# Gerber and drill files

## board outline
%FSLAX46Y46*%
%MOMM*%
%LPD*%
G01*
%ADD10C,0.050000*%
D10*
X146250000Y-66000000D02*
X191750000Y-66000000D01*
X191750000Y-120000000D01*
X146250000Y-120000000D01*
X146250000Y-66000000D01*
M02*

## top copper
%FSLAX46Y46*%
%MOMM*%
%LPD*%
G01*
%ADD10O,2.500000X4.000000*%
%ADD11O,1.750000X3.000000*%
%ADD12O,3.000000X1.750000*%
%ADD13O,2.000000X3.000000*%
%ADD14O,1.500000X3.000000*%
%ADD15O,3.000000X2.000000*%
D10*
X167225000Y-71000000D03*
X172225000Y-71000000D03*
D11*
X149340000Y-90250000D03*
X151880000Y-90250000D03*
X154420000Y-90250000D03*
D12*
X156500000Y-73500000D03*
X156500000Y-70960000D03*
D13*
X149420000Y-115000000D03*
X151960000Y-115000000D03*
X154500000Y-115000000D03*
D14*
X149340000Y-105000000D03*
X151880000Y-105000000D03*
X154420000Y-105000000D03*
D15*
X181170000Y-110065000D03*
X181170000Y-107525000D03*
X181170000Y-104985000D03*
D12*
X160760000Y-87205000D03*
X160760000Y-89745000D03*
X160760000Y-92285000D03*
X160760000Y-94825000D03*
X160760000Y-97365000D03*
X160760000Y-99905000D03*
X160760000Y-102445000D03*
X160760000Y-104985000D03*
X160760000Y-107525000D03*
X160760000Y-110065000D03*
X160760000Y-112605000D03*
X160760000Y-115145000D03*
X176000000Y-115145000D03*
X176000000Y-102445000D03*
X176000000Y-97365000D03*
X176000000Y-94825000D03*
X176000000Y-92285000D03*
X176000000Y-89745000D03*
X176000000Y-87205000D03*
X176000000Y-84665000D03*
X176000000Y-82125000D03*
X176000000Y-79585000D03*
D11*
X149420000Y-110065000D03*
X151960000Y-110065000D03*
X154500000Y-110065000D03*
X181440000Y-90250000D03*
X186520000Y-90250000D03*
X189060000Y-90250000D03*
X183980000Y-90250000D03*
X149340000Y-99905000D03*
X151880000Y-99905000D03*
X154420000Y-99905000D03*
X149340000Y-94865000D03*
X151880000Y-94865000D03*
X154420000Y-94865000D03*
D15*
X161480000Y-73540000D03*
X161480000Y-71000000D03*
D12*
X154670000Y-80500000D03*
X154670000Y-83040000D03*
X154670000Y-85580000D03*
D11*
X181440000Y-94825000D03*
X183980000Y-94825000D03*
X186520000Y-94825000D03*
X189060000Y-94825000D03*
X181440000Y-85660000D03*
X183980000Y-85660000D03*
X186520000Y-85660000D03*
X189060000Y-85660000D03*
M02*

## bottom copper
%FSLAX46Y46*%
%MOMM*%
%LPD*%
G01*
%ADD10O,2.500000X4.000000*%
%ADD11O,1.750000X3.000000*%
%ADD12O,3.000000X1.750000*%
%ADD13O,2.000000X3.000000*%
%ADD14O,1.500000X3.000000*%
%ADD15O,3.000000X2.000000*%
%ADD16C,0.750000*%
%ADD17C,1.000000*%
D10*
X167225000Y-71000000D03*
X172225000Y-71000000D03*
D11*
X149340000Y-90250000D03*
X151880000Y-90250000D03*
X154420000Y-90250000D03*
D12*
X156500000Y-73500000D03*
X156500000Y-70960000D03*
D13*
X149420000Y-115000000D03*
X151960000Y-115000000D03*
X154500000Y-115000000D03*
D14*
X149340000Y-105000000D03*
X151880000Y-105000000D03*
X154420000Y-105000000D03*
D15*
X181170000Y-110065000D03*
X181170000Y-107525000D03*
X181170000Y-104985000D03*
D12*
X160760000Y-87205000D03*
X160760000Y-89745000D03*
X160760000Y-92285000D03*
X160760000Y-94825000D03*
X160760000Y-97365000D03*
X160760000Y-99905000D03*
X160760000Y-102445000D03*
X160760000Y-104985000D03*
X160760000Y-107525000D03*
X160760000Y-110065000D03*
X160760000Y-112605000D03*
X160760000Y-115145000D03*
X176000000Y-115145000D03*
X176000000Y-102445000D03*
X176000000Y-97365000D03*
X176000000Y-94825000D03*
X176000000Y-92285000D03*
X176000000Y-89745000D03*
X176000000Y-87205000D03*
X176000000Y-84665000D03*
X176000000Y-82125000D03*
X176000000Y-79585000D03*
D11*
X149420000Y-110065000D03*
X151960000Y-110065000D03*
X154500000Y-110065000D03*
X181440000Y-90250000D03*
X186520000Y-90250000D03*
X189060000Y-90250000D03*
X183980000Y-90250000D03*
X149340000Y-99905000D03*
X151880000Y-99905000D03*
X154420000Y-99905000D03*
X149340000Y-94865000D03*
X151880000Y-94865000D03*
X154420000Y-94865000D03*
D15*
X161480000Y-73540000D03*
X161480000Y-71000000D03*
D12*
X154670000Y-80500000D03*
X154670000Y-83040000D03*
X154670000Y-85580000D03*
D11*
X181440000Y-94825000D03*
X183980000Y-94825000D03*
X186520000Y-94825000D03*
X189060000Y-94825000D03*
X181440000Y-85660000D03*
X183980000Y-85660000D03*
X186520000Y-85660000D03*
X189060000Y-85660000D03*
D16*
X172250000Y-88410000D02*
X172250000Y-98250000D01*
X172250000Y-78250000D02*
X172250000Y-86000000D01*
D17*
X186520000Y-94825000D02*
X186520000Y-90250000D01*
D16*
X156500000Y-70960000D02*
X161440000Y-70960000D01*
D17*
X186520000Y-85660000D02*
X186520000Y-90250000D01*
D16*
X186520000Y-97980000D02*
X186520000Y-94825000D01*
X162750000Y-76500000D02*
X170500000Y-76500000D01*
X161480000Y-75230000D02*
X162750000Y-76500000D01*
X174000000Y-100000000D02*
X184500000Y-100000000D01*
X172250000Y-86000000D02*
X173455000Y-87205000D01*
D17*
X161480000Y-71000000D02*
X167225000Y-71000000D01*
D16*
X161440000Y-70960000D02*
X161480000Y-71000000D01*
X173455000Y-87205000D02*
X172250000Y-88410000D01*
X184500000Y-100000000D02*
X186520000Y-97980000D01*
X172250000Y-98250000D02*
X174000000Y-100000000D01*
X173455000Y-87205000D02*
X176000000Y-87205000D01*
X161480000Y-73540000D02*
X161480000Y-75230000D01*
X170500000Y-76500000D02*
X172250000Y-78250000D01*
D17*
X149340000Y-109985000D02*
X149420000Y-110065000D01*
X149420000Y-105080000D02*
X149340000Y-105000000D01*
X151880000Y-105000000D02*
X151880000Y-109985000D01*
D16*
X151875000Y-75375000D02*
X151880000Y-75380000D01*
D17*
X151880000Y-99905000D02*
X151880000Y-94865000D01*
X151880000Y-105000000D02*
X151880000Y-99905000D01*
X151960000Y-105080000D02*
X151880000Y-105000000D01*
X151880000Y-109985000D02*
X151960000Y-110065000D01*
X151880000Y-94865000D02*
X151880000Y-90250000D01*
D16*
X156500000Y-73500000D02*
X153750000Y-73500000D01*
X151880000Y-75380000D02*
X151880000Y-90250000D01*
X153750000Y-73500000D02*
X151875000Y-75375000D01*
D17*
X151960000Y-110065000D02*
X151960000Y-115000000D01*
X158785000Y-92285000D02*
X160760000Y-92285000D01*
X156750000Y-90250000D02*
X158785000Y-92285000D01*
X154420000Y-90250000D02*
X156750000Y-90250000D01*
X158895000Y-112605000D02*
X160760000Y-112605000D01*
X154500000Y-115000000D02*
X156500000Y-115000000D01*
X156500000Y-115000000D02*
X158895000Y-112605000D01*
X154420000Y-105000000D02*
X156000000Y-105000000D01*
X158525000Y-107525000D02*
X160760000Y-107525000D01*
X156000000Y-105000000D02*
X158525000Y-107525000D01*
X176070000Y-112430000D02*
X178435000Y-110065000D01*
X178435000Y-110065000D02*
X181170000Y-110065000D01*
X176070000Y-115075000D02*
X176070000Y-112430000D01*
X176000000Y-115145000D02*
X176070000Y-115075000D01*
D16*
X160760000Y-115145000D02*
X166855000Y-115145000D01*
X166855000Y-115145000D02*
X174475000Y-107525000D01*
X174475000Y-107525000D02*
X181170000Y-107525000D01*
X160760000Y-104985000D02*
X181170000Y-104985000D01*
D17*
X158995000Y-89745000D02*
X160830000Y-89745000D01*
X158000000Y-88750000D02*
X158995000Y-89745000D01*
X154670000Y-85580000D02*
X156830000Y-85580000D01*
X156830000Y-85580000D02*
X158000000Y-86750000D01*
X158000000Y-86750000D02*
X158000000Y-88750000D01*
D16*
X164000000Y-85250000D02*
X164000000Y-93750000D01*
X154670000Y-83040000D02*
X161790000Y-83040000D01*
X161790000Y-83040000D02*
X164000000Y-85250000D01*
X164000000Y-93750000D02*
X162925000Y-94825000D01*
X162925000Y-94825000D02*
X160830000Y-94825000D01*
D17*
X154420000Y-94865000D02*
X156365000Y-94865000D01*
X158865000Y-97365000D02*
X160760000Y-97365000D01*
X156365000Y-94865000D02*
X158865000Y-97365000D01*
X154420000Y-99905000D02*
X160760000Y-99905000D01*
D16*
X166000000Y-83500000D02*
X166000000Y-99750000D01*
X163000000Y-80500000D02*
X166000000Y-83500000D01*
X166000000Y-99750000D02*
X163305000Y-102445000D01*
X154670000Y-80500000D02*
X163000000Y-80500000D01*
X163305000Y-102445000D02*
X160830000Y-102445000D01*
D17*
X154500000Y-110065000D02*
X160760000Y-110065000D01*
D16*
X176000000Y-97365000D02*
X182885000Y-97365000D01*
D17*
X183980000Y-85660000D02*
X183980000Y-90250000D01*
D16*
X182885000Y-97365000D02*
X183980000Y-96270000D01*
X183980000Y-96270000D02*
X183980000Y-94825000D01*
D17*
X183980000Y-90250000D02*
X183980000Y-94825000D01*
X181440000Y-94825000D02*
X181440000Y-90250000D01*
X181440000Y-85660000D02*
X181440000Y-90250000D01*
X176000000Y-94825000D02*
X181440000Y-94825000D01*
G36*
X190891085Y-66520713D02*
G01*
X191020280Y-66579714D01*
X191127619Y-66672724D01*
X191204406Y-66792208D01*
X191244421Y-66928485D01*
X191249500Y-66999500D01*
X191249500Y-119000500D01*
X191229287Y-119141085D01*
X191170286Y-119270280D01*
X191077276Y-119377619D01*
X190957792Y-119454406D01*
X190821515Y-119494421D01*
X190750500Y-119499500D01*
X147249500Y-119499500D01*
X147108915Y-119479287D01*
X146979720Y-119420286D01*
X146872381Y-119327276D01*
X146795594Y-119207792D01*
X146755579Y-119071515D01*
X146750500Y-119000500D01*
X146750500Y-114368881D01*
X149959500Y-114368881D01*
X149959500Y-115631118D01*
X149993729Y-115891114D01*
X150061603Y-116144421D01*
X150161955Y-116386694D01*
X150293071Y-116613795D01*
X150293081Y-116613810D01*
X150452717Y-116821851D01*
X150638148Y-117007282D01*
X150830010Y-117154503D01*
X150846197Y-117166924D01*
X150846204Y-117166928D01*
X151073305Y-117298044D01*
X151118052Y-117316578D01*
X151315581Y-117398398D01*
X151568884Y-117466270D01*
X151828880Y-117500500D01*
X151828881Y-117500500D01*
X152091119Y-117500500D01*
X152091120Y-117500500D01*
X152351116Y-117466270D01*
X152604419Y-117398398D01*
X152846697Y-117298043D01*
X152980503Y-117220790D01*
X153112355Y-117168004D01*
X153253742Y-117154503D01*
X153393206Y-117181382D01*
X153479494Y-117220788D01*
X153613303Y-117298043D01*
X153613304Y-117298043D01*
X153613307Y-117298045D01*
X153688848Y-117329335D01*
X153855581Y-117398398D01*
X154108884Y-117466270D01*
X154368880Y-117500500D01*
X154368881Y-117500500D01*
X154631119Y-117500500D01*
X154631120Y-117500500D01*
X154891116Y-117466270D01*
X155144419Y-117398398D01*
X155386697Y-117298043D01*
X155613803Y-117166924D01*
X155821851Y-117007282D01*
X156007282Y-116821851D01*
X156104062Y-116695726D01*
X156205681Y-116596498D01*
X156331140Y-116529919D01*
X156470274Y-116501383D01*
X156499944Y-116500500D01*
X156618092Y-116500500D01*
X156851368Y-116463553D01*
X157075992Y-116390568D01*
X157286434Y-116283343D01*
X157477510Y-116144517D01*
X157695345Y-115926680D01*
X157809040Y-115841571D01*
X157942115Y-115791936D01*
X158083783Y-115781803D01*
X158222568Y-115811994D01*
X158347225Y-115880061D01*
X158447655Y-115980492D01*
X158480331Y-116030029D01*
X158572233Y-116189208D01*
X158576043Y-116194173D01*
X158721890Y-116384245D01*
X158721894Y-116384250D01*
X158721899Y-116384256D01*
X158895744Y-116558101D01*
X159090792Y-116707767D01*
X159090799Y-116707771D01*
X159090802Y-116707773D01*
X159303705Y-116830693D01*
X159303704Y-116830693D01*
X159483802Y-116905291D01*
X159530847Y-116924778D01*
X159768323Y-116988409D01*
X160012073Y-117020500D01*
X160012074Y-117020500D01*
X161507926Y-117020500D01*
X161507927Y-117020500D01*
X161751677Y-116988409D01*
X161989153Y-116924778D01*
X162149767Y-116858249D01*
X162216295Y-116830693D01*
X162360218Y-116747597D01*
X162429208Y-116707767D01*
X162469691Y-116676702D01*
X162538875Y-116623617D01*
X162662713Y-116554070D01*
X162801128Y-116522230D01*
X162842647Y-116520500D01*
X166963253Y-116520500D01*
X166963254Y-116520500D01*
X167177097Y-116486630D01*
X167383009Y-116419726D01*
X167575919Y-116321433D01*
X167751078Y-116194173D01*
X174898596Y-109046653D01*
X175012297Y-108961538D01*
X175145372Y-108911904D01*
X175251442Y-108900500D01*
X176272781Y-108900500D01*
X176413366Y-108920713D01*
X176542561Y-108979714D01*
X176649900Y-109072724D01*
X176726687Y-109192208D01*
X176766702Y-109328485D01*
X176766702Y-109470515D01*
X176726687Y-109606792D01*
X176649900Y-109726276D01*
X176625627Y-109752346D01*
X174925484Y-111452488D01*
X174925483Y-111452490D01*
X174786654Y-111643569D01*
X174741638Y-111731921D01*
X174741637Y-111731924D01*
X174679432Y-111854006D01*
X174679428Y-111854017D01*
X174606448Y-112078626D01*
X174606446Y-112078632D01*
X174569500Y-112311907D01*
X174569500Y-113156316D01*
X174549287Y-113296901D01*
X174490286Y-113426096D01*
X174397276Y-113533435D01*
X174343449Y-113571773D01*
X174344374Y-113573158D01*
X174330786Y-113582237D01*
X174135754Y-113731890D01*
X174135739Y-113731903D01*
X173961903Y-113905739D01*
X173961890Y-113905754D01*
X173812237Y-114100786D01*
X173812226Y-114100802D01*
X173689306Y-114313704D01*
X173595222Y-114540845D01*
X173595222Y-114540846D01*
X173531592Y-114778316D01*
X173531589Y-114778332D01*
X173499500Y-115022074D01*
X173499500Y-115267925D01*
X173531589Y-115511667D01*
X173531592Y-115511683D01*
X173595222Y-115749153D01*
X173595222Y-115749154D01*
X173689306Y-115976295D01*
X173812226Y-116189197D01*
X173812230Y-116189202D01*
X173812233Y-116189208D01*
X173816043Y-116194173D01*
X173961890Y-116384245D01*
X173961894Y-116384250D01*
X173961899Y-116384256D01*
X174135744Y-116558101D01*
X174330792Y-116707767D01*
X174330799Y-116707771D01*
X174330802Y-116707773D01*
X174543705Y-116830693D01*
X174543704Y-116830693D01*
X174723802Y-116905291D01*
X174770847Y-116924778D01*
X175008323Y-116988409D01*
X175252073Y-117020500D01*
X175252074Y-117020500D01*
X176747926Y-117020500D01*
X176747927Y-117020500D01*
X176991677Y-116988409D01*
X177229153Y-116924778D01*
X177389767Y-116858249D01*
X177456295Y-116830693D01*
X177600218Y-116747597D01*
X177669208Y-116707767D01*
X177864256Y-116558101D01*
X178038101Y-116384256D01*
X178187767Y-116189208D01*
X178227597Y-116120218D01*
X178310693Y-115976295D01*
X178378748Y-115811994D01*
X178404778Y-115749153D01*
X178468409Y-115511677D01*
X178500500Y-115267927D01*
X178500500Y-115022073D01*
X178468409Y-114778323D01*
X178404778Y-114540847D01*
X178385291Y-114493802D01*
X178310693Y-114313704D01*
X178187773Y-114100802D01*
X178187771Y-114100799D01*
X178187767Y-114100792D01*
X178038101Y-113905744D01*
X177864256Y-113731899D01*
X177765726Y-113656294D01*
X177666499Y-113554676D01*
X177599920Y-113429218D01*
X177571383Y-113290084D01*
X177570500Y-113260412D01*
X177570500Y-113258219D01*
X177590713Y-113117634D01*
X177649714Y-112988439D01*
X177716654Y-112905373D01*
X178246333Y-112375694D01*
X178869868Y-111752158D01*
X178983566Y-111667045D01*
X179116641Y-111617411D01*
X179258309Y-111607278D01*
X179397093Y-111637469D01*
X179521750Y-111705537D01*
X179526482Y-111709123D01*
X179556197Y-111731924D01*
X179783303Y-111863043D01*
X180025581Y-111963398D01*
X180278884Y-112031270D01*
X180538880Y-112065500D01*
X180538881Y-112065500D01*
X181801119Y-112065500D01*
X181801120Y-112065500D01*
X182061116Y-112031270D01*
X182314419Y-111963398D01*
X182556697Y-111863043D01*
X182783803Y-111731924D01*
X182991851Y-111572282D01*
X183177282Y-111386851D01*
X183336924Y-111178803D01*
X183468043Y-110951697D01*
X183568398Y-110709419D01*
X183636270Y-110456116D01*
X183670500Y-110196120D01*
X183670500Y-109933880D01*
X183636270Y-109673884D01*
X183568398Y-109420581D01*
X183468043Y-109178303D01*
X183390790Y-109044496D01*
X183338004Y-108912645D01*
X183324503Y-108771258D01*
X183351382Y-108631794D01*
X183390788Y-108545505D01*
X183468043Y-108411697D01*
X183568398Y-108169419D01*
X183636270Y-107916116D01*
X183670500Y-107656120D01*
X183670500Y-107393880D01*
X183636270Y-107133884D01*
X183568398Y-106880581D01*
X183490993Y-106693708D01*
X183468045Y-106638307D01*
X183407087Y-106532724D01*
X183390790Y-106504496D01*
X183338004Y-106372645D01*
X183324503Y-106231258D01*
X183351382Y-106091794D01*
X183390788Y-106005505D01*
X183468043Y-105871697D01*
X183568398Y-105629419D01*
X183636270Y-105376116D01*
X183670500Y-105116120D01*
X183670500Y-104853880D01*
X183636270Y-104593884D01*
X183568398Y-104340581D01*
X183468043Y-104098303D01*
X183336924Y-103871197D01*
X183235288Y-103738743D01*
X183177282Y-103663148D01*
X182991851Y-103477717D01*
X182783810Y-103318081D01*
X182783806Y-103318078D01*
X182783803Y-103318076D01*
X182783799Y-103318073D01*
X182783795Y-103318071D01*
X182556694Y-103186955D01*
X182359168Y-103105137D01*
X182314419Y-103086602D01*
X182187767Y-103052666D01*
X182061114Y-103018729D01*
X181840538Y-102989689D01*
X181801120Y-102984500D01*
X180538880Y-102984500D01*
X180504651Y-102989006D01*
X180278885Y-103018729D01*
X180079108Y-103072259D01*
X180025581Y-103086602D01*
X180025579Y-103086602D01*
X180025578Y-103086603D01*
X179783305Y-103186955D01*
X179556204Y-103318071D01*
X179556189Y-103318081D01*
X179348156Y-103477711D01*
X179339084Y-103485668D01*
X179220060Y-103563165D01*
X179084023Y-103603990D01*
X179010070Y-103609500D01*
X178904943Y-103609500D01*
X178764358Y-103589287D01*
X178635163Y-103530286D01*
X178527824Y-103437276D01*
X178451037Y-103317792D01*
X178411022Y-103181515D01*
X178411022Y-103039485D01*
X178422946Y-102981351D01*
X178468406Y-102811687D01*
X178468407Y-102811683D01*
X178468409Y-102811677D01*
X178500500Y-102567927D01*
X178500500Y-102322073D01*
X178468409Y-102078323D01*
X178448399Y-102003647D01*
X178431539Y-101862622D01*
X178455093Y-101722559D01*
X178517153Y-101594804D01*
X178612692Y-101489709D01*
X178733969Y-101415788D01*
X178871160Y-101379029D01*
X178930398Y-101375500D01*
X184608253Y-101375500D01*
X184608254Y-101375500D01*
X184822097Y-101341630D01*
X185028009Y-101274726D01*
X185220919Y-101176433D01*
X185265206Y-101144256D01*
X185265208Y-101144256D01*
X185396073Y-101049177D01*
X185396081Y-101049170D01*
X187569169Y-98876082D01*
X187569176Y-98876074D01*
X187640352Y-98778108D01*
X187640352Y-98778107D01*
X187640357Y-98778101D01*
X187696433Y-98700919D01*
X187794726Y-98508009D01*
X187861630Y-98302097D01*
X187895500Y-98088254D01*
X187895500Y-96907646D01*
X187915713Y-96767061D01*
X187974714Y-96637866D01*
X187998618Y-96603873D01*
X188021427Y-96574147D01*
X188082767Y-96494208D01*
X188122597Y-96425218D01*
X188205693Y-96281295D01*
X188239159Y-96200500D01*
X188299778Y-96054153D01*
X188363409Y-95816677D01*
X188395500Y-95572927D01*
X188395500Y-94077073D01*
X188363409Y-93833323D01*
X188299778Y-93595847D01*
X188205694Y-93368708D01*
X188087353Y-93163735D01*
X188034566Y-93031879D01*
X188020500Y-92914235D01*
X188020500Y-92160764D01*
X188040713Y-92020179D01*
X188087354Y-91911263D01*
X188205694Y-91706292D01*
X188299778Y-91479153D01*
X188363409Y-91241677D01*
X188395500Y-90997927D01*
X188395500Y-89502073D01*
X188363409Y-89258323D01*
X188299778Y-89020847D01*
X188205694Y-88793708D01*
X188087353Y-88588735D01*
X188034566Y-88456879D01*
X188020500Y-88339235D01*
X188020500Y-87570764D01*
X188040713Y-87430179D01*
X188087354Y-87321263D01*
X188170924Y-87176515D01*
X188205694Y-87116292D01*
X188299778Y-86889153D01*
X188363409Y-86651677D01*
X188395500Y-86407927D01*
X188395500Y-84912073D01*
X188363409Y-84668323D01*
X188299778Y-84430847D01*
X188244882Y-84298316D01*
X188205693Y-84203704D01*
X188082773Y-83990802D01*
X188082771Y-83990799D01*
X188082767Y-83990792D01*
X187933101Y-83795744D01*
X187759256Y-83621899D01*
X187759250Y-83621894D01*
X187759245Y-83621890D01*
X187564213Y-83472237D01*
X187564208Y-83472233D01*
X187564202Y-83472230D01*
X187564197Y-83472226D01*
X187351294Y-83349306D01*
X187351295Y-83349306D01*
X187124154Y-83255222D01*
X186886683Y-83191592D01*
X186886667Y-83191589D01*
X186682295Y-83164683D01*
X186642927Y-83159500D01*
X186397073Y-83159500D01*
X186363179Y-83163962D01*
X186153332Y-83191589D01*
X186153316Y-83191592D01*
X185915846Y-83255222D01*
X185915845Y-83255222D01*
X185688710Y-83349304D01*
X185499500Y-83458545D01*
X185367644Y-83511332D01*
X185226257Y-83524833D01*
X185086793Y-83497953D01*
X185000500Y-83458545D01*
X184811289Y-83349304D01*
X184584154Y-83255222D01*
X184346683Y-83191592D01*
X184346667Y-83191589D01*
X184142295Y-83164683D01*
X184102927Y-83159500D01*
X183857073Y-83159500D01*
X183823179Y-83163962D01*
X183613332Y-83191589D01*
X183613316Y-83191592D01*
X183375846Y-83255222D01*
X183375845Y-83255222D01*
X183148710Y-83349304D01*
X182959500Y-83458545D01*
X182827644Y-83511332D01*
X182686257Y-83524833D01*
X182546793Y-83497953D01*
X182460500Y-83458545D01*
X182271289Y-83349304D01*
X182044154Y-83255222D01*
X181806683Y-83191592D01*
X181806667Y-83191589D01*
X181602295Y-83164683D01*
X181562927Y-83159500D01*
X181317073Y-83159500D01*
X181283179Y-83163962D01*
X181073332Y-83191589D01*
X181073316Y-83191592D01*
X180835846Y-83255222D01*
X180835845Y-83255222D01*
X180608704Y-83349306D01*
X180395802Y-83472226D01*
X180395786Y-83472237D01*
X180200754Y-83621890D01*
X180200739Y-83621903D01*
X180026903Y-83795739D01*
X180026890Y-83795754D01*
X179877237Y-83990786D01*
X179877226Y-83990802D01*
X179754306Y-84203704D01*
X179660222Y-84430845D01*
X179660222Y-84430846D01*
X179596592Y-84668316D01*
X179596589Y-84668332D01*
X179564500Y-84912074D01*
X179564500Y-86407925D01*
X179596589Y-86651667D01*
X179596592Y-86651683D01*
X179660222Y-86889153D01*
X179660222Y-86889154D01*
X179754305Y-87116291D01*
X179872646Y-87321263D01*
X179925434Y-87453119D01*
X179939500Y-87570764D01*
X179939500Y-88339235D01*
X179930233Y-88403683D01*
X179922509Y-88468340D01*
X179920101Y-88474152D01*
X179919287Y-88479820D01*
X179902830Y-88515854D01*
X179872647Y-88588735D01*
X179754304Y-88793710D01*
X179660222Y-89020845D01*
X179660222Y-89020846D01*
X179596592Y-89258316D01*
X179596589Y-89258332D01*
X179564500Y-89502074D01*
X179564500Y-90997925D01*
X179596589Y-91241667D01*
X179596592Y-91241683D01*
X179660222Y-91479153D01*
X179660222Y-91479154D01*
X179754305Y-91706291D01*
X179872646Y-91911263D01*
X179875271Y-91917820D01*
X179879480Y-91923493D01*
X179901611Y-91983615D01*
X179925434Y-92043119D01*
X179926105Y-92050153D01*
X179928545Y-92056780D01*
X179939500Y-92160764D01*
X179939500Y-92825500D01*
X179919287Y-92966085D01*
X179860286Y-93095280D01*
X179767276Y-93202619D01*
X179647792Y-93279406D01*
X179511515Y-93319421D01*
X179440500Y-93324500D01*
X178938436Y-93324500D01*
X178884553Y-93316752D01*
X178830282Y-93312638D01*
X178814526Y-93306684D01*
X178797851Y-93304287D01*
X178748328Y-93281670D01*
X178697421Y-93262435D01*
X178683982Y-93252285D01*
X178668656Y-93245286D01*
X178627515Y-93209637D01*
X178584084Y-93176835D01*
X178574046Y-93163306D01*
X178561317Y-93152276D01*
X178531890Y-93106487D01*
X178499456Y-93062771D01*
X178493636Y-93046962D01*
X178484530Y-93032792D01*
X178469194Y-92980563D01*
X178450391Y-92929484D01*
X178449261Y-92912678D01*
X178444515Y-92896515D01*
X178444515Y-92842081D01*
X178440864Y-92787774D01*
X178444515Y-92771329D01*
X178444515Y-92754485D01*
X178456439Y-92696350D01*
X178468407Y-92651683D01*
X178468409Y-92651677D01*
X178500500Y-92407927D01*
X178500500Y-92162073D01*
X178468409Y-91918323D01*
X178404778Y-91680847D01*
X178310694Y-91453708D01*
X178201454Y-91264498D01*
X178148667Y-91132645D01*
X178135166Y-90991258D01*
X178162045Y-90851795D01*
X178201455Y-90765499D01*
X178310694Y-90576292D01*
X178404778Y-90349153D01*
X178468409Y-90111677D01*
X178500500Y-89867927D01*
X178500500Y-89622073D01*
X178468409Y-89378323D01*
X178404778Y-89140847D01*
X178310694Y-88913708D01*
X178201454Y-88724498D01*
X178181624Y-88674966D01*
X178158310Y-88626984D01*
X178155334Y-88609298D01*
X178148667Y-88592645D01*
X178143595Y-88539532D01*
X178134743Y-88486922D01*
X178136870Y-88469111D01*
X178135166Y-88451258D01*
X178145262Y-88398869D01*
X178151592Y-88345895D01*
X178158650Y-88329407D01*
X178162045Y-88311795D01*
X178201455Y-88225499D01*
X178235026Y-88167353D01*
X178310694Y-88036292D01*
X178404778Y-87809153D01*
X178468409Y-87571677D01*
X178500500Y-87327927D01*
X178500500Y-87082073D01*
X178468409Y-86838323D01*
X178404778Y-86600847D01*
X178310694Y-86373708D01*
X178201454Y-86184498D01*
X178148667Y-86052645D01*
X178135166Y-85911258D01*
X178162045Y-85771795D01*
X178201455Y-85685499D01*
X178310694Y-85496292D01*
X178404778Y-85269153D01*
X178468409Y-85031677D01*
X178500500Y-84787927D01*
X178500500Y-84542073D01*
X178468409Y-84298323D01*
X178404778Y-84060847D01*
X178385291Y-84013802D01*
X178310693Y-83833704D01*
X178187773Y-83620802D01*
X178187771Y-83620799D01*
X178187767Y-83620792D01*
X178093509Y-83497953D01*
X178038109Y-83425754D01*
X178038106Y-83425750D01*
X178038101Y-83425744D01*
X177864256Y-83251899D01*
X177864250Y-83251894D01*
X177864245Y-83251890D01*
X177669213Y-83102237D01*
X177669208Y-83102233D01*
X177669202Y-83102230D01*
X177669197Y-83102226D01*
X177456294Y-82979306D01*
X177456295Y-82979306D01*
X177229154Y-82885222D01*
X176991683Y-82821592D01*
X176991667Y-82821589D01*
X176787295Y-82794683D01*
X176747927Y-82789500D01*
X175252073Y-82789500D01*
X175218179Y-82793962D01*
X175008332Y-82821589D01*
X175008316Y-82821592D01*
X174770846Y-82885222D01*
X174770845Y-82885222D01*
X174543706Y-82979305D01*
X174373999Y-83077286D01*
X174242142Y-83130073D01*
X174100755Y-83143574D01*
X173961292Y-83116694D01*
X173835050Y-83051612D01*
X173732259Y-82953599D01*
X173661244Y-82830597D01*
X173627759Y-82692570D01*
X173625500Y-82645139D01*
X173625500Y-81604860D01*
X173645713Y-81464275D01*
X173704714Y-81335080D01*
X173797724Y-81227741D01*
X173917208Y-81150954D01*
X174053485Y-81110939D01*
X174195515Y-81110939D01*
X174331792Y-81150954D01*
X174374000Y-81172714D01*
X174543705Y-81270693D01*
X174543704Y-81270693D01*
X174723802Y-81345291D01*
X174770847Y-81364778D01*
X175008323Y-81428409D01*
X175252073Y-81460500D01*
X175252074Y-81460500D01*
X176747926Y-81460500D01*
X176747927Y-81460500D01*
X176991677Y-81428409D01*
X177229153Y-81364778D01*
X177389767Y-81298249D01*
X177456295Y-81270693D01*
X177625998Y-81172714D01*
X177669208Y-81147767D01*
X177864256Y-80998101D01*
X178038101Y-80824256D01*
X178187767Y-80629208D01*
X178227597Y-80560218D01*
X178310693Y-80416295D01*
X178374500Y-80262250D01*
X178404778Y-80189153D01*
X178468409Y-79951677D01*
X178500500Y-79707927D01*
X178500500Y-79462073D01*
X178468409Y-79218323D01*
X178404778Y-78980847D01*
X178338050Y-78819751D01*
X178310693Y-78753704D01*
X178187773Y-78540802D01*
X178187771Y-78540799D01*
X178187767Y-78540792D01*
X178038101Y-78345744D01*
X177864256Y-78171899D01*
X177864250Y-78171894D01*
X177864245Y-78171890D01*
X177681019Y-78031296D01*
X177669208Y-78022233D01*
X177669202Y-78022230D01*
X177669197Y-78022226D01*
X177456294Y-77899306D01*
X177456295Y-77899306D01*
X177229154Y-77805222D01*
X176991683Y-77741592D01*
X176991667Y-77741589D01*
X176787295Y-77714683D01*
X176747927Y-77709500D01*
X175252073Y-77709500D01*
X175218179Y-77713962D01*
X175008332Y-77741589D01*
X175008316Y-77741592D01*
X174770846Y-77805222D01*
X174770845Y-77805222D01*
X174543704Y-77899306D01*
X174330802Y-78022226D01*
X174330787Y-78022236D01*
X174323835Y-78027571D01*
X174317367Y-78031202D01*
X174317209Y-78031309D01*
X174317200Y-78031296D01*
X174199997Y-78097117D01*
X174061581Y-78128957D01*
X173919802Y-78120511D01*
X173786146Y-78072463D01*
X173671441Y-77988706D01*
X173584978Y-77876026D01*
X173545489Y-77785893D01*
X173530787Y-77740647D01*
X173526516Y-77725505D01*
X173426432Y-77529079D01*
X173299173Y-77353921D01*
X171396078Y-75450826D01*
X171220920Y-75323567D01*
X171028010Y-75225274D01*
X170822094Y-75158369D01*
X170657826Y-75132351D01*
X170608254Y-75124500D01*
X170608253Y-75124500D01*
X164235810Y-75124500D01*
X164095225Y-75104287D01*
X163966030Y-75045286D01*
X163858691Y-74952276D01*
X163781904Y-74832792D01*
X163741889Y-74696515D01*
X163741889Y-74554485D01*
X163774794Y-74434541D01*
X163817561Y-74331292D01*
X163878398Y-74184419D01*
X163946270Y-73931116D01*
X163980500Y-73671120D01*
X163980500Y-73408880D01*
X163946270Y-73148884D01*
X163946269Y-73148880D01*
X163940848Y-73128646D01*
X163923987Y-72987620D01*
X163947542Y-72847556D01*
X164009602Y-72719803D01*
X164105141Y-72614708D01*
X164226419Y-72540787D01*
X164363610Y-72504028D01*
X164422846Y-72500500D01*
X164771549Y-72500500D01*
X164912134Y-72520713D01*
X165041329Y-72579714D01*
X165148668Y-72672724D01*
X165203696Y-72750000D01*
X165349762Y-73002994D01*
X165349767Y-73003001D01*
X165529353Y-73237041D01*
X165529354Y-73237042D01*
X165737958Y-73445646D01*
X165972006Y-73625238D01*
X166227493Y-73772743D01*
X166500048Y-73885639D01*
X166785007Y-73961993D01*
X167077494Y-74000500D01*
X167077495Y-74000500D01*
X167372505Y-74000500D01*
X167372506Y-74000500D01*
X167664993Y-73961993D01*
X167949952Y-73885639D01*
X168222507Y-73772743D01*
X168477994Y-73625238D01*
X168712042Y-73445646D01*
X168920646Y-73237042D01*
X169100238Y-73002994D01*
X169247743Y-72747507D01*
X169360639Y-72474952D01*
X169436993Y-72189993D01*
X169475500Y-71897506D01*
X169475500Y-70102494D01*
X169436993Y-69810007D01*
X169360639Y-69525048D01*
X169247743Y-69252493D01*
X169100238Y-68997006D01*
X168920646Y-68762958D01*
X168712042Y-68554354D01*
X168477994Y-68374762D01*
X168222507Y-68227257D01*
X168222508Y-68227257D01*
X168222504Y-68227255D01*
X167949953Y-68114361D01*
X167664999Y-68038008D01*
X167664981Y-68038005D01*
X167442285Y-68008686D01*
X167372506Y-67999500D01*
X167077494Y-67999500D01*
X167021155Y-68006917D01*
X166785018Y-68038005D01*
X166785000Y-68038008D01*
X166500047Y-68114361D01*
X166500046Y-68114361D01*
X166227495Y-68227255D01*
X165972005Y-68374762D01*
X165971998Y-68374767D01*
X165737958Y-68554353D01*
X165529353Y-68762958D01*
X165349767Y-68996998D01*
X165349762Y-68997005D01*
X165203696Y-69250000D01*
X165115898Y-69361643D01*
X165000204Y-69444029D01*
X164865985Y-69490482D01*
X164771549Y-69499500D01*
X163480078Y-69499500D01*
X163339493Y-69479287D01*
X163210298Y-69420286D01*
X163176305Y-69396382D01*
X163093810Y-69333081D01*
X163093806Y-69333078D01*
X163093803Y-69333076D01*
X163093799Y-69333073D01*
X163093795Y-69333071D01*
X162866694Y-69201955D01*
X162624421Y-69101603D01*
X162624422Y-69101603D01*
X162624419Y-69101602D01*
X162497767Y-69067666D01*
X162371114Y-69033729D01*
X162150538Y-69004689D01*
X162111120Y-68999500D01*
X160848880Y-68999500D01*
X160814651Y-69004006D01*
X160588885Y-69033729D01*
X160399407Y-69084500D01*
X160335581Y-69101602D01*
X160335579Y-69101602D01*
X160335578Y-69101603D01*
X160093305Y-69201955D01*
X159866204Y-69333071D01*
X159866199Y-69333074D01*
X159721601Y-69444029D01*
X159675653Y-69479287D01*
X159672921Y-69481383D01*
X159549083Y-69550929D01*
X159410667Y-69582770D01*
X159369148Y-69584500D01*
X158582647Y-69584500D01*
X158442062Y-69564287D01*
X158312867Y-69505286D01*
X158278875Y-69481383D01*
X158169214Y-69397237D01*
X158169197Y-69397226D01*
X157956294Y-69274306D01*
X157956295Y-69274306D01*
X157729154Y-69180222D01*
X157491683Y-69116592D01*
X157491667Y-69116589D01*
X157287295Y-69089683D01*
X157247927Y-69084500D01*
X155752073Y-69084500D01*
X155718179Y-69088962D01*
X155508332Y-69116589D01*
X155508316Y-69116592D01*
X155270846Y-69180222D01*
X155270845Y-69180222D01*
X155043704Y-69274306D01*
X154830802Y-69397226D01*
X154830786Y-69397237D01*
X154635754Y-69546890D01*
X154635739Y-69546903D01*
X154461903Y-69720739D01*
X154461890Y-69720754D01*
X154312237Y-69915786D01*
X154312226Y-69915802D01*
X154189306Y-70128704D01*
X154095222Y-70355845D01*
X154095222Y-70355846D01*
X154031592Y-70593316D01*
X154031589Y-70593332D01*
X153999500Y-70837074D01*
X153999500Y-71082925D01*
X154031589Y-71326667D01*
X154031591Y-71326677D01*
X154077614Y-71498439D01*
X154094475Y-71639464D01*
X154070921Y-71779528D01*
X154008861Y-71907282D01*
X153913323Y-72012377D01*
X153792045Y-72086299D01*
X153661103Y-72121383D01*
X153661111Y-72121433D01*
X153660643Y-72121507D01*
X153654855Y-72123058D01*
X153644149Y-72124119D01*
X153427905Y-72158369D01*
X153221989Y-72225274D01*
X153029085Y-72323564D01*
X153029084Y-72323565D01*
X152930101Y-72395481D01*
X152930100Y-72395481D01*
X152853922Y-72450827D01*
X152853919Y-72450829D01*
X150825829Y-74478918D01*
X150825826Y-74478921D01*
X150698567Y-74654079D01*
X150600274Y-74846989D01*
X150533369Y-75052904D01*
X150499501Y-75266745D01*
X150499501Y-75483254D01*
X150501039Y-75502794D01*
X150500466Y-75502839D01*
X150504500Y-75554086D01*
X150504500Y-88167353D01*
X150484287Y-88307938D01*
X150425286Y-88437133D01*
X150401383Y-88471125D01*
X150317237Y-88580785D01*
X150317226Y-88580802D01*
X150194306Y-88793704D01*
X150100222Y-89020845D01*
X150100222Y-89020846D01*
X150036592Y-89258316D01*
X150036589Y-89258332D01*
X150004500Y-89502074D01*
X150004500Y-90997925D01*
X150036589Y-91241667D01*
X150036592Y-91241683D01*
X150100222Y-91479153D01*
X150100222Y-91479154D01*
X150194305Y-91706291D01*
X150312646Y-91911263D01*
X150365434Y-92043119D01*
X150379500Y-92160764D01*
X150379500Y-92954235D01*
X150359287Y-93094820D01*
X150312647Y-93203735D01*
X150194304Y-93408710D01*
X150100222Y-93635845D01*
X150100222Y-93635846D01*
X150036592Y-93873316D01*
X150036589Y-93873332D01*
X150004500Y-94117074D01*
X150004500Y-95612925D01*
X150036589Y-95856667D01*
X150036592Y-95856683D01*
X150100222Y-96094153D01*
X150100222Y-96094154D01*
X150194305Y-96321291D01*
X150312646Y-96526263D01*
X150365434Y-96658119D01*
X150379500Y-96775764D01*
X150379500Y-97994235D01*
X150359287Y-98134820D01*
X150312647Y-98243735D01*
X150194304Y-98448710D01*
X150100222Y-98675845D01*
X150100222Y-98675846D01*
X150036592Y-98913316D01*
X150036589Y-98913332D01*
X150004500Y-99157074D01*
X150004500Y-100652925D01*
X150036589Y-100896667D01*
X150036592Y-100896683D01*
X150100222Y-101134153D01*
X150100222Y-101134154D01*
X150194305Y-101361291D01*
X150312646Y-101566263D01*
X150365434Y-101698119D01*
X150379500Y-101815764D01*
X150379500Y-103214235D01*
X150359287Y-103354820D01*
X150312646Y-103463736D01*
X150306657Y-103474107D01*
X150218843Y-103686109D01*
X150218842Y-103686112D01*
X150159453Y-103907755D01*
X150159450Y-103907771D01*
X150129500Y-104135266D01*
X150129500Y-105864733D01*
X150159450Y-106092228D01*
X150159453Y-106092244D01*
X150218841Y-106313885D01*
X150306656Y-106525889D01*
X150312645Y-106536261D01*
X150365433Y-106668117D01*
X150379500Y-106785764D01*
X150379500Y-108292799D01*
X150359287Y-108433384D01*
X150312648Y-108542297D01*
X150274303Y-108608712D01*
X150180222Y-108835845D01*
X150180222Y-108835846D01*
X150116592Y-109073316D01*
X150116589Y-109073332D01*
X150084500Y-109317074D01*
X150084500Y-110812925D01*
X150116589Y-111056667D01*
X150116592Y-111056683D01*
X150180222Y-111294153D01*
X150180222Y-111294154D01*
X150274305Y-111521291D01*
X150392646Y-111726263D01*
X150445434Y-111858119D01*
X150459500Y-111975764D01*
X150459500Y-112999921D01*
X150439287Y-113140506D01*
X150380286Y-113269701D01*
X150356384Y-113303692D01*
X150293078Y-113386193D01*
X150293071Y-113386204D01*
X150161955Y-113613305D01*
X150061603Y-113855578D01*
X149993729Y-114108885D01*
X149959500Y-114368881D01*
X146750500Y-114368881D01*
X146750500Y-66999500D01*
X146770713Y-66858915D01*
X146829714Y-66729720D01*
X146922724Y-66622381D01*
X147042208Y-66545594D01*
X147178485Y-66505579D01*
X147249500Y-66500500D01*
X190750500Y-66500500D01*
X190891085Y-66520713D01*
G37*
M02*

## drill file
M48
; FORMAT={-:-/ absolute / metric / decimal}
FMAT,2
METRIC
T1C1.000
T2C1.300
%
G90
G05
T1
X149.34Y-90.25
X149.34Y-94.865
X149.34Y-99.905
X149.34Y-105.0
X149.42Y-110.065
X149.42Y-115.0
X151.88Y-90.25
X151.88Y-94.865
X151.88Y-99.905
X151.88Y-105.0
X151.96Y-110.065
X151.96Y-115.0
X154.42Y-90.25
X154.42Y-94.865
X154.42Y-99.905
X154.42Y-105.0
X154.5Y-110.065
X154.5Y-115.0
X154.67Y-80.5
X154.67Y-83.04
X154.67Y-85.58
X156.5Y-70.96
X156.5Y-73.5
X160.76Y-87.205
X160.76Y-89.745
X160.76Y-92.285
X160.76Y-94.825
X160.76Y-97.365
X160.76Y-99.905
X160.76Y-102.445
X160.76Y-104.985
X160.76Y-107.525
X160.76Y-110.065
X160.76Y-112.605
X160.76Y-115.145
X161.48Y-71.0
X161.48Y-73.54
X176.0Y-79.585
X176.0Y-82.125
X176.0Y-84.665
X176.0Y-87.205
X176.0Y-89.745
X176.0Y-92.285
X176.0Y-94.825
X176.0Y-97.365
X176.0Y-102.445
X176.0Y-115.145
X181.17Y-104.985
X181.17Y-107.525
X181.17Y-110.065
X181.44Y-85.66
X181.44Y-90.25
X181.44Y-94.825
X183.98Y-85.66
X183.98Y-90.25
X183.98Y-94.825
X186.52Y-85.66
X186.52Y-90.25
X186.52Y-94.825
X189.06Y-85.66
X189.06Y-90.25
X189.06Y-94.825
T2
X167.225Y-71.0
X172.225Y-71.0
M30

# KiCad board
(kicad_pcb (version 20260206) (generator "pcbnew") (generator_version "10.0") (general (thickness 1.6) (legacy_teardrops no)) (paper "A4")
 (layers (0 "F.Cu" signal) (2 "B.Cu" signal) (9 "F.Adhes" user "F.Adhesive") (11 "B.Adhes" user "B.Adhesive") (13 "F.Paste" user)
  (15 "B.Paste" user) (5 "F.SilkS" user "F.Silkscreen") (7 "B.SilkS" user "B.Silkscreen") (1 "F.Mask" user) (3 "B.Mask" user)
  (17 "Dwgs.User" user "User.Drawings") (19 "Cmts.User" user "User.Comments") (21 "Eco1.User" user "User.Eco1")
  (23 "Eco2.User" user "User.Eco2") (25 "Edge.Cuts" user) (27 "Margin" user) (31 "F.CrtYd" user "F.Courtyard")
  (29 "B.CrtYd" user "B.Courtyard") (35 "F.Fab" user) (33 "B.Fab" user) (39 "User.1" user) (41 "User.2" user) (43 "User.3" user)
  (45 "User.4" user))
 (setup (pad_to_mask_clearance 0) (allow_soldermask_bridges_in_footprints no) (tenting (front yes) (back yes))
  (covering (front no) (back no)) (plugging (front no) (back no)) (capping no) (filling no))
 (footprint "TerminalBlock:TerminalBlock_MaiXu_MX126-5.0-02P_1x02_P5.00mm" (layer "F.Cu") (at 167.225 71)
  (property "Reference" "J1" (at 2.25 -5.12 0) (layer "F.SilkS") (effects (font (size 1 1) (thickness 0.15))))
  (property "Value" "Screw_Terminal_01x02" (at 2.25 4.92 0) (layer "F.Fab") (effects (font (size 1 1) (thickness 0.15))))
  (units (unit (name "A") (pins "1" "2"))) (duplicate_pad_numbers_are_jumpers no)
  (pad "1" thru_hole oval (at 0 0) (size 2.5 4) (drill 1.3) (layers "*.Cu" "*.Mask") (remove_unused_layers no) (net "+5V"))
  (pad "2" thru_hole oval (at 5 0) (size 2.5 4) (drill 1.3) (layers "*.Cu" "*.Mask") (remove_unused_layers no) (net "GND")))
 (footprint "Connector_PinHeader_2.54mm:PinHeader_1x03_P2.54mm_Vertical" (layer "F.Cu") (at 149.34 90.25 90)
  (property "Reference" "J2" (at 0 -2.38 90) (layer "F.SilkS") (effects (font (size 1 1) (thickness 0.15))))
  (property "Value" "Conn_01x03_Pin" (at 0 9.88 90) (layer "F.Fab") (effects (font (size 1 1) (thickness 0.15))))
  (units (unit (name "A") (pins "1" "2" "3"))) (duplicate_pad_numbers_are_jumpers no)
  (pad "1" thru_hole oval (at 0 0 90) (size 3 1.75) (drill 1) (layers "*.Cu" "*.Mask") (remove_unused_layers no) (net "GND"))
  (pad "2" thru_hole oval (at 0 2.54 90) (size 3 1.75) (drill 1) (layers "*.Cu" "*.Mask") (remove_unused_layers no) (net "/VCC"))
  (pad "3" thru_hole oval (at 0 5.08 90) (size 3 1.75) (drill 1) (layers "*.Cu" "*.Mask") (remove_unused_layers no) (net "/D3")))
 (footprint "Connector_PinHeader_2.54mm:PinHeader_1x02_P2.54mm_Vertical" (layer "F.Cu") (at 156.5 73.5 180)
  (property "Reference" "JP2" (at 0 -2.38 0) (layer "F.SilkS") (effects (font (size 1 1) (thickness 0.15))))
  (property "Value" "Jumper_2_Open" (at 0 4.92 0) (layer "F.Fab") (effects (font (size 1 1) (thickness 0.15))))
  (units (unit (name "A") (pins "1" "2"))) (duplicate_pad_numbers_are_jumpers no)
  (pad "1" thru_hole oval (at 0 0 180) (size 3 1.75) (drill 1) (layers "*.Cu" "*.Mask") (remove_unused_layers no) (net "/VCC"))
  (pad "2" thru_hole oval (at 0 2.54 180) (size 3 1.75) (drill 1) (layers "*.Cu" "*.Mask") (remove_unused_layers no) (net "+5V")))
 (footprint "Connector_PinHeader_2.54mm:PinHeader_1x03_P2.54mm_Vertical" (layer "F.Cu") (at 149.42 115 90)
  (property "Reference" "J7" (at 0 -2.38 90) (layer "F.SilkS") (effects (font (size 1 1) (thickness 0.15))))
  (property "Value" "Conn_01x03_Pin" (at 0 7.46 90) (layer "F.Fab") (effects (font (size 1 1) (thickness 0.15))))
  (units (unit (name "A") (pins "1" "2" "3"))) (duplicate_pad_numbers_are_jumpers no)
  (pad "1" thru_hole oval (at 0 0 90) (size 3 2) (drill 1) (layers "*.Cu" "*.Mask") (remove_unused_layers no) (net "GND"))
  (pad "2" thru_hole oval (at 0 2.54 90) (size 3 2) (drill 1) (layers "*.Cu" "*.Mask") (remove_unused_layers no) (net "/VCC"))
  (pad "3" thru_hole oval (at 0 5.08 90) (size 3 2) (drill 1) (layers "*.Cu" "*.Mask") (remove_unused_layers no) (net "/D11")))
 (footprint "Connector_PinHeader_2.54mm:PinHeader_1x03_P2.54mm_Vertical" (layer "F.Cu") (at 149.34 105 90)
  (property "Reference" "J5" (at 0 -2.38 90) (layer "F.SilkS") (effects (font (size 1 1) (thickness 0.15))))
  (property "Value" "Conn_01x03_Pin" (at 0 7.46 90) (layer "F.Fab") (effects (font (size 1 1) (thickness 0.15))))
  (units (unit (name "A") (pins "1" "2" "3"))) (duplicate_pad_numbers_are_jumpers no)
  (pad "1" thru_hole oval (at 0 0 90) (size 3 1.5) (drill 1) (layers "*.Cu" "*.Mask") (remove_unused_layers no) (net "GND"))
  (pad "2" thru_hole oval (at 0 2.54 90) (size 3 1.5) (drill 1) (layers "*.Cu" "*.Mask") (remove_unused_layers no) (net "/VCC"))
  (pad "3" thru_hole oval (at 0 5.08 90) (size 3 1.5) (drill 1) (layers "*.Cu" "*.Mask") (remove_unused_layers no) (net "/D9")))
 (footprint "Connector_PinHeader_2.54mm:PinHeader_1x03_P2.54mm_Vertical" (layer "F.Cu") (at 181.17 110.065 180)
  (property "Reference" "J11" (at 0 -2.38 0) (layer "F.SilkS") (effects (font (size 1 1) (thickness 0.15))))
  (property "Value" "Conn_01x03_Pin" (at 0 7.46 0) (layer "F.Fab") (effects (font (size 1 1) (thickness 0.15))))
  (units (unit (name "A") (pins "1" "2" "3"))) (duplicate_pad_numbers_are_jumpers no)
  (pad "1" thru_hole oval (at 0 0 180) (size 3 2) (drill 1) (layers "*.Cu" "*.Mask") (remove_unused_layers no) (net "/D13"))
  (pad "2" thru_hole oval (at 0 2.54 180) (size 3 2) (drill 1) (layers "*.Cu" "*.Mask") (remove_unused_layers no) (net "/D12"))
  (pad "3" thru_hole oval (at 0 5.08 180) (size 3 2) (drill 1) (layers "*.Cu" "*.Mask") (remove_unused_layers no) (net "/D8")))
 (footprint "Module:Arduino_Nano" (layer "F.Cu") (at 160.76 79.585)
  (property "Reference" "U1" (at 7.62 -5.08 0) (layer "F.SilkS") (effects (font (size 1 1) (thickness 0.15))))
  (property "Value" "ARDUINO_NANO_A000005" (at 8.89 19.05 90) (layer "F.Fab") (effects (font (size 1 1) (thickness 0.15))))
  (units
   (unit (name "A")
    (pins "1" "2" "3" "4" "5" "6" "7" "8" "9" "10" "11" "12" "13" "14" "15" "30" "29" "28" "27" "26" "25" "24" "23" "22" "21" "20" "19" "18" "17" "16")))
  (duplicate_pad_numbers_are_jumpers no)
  (pad "4" thru_hole oval (at 0 7.62) (size 3 1.75) (drill 1) (layers "*.Cu" "*.Mask") (remove_unused_layers no)
   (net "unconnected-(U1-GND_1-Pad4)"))
  (pad "5" thru_hole oval (at 0 10.16) (size 3 1.75) (drill 1) (layers "*.Cu" "*.Mask") (remove_unused_layers no) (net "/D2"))
  (pad "6" thru_hole oval (at 0 12.7) (size 3 1.75) (drill 1) (layers "*.Cu" "*.Mask") (remove_unused_layers no) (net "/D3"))
  (pad "7" thru_hole oval (at 0 15.24) (size 3 1.75) (drill 1) (layers "*.Cu" "*.Mask") (remove_unused_layers no) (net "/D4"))
  (pad "8" thru_hole oval (at 0 17.78) (size 3 1.75) (drill 1) (layers "*.Cu" "*.Mask") (remove_unused_layers no) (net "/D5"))
  (pad "9" thru_hole oval (at 0 20.32) (size 3 1.75) (drill 1) (layers "*.Cu" "*.Mask") (remove_unused_layers no) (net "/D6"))
  (pad "10" thru_hole oval (at 0 22.86) (size 3 1.75) (drill 1) (layers "*.Cu" "*.Mask") (remove_unused_layers no) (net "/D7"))
  (pad "11" thru_hole oval (at 0 25.4) (size 3 1.75) (drill 1) (layers "*.Cu" "*.Mask") (remove_unused_layers no) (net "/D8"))
  (pad "12" thru_hole oval (at 0 27.94) (size 3 1.75) (drill 1) (layers "*.Cu" "*.Mask") (remove_unused_layers no) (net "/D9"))
  (pad "13" thru_hole oval (at 0 30.48) (size 3 1.75) (drill 1) (layers "*.Cu" "*.Mask") (remove_unused_layers no) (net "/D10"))
  (pad "14" thru_hole oval (at 0 33.02) (size 3 1.75) (drill 1) (layers "*.Cu" "*.Mask") (remove_unused_layers no) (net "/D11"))
  (pad "15" thru_hole oval (at 0 35.56) (size 3 1.75) (drill 1) (layers "*.Cu" "*.Mask") (remove_unused_layers no) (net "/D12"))
  (pad "16" thru_hole oval (at 15.24 35.56) (size 3 1.75) (drill 1) (layers "*.Cu" "*.Mask") (remove_unused_layers no) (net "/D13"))
  (pad "21" thru_hole oval (at 15.24 22.86) (size 3 1.75) (drill 1) (layers "*.Cu" "*.Mask") (remove_unused_layers no)
   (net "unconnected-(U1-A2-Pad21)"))
  (pad "23" thru_hole oval (at 15.24 17.78) (size 3 1.75) (drill 1) (layers "*.Cu" "*.Mask") (remove_unused_layers no) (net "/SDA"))
  (pad "24" thru_hole oval (at 15.24 15.24) (size 3 1.75) (drill 1) (layers "*.Cu" "*.Mask") (remove_unused_layers no) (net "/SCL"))
  (pad "25" thru_hole oval (at 15.24 12.7) (size 3 1.75) (drill 1) (layers "*.Cu" "*.Mask") (remove_unused_layers no)
   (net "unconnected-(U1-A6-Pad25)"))
  (pad "26" thru_hole oval (at 15.24 10.16) (size 3 1.75) (drill 1) (layers "*.Cu" "*.Mask") (remove_unused_layers no)
   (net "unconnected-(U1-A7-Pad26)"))
  (pad "27" thru_hole oval (at 15.24 7.62) (size 3 1.75) (drill 1) (layers "*.Cu" "*.Mask") (remove_unused_layers no) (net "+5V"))
  (pad "28" thru_hole oval (at 15.24 5.08) (size 3 1.75) (drill 1) (layers "*.Cu" "*.Mask") (remove_unused_layers no)
   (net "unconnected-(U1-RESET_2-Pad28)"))
  (pad "29" thru_hole oval (at 15.24 2.54) (size 3 1.75) (drill 1) (layers "*.Cu" "*.Mask") (remove_unused_layers no) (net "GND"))
  (pad "30" thru_hole oval (at 15.24 0) (size 3 1.75) (drill 1) (layers "*.Cu" "*.Mask") (remove_unused_layers no)
   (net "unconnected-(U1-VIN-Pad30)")))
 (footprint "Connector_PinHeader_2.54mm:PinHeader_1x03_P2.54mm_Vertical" (layer "F.Cu") (at 149.42 110.065 90)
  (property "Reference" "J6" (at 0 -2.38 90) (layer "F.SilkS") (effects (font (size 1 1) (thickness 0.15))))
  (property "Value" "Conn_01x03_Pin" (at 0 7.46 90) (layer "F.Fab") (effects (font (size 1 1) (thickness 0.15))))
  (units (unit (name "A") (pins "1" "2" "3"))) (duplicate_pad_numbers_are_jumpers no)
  (pad "1" thru_hole oval (at 0 0 90) (size 3 1.75) (drill 1) (layers "*.Cu" "*.Mask") (remove_unused_layers no) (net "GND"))
  (pad "2" thru_hole oval (at 0 2.54 90) (size 3 1.75) (drill 1) (layers "*.Cu" "*.Mask") (remove_unused_layers no) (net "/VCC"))
  (pad "3" thru_hole oval (at 0 5.08 90) (size 3 1.75) (drill 1) (layers "*.Cu" "*.Mask") (remove_unused_layers no) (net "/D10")))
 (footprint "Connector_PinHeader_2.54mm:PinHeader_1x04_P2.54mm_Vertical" (layer "F.Cu") (at 181.44 90.25 90)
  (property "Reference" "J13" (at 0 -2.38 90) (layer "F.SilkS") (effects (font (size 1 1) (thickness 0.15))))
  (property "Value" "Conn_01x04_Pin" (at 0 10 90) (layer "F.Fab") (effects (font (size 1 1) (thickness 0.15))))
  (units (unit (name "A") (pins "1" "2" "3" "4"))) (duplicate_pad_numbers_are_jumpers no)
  (pad "1" thru_hole oval (at 0 0 90) (size 3 1.75) (drill 1) (layers "*.Cu" "*.Mask") (remove_unused_layers no) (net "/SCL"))
  (pad "3" thru_hole oval (at 0 5.08 90) (size 3 1.75) (drill 1) (layers "*.Cu" "*.Mask") (remove_unused_layers no) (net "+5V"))
  (pad "4" thru_hole oval (at 0 7.62 90) (size 3 1.75) (drill 1) (layers "*.Cu" "*.Mask") (remove_unused_layers no) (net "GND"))
  (pad "E" thru_hole oval (at 0 2.54 90) (size 3 1.75) (drill 1) (layers "*.Cu" "*.Mask") (remove_unused_layers no)))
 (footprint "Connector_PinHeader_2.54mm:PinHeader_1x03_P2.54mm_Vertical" (layer "F.Cu") (at 149.34 99.905 90)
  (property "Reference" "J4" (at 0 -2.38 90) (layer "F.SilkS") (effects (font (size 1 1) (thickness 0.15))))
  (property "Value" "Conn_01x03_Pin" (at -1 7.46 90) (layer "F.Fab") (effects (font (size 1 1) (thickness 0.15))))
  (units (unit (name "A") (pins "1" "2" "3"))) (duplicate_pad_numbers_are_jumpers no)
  (pad "1" thru_hole oval (at 0 0 90) (size 3 1.75) (drill 1) (layers "*.Cu" "*.Mask") (remove_unused_layers no) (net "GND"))
  (pad "2" thru_hole oval (at 0 2.54 90) (size 3 1.75) (drill 1) (layers "*.Cu" "*.Mask") (remove_unused_layers no) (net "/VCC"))
  (pad "3" thru_hole oval (at 0 5.08 90) (size 3 1.75) (drill 1) (layers "*.Cu" "*.Mask") (remove_unused_layers no) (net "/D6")))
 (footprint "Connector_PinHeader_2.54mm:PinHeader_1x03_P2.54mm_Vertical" (layer "F.Cu") (at 149.34 94.865 90)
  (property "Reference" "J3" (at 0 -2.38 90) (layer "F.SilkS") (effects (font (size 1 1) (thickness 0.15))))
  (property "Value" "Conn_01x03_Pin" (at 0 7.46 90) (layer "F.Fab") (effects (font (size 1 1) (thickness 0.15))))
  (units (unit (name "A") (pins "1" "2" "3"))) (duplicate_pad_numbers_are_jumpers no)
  (pad "1" thru_hole oval (at 0 0 90) (size 3 1.75) (drill 1) (layers "*.Cu" "*.Mask") (remove_unused_layers no) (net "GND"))
  (pad "2" thru_hole oval (at 0 2.54 90) (size 3 1.75) (drill 1) (layers "*.Cu" "*.Mask") (remove_unused_layers no) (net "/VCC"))
  (pad "3" thru_hole oval (at 0 5.08 90) (size 3 1.75) (drill 1) (layers "*.Cu" "*.Mask") (remove_unused_layers no) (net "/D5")))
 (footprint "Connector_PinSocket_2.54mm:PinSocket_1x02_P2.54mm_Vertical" (layer "F.Cu") (at 161.48 73.54 180)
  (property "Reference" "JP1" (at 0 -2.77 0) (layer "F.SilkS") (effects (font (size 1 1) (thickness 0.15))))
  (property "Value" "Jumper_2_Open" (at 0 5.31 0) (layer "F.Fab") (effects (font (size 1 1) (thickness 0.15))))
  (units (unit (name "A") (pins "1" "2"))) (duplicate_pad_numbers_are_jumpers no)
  (pad "1" thru_hole oval (at 0 0 180) (size 3 2) (drill 1) (layers "*.Cu" "*.Mask") (remove_unused_layers no) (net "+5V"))
  (pad "2" thru_hole oval (at 0 2.54 180) (size 3 2) (drill 1) (layers "*.Cu" "*.Mask") (remove_unused_layers no) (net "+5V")))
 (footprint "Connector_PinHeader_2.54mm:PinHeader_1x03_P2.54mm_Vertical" (layer "F.Cu") (at 154.67 80.5)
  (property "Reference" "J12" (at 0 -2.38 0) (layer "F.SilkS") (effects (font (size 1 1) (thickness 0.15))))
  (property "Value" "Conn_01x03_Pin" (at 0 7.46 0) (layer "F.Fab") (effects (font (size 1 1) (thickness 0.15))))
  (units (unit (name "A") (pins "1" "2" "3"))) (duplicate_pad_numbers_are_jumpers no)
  (pad "1" thru_hole oval (at 0 0) (size 3 1.75) (drill 1) (layers "*.Cu" "*.Mask") (remove_unused_layers no) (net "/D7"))
  (pad "2" thru_hole oval (at 0 2.54) (size 3 1.75) (drill 1) (layers "*.Cu" "*.Mask") (remove_unused_layers no) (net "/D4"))
  (pad "3" thru_hole oval (at 0 5.08) (size 3 1.75) (drill 1) (layers "*.Cu" "*.Mask") (remove_unused_layers no) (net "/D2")))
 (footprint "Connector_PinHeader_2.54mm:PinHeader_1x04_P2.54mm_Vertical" (layer "F.Cu") (at 181.44 94.825 90)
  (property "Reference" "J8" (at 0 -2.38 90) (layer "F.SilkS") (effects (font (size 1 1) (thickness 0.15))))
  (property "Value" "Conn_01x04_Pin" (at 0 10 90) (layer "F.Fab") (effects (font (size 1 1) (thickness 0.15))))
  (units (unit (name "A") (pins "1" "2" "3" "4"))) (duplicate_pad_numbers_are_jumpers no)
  (pad "1" thru_hole oval (at 0 0 90) (size 3 1.75) (drill 1) (layers "*.Cu" "*.Mask") (remove_unused_layers no) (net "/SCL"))
  (pad "2" thru_hole oval (at 0 2.54 90) (size 3 1.75) (drill 1) (layers "*.Cu" "*.Mask") (remove_unused_layers no) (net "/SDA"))
  (pad "3" thru_hole oval (at 0 5.08 90) (size 3 1.75) (drill 1) (layers "*.Cu" "*.Mask") (remove_unused_layers no) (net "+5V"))
  (pad "4" thru_hole oval (at 0 7.62 90) (size 3 1.75) (drill 1) (layers "*.Cu" "*.Mask") (remove_unused_layers no) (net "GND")))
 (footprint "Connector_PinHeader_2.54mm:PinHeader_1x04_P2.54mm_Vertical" (layer "F.Cu") (at 181.44 85.66 90)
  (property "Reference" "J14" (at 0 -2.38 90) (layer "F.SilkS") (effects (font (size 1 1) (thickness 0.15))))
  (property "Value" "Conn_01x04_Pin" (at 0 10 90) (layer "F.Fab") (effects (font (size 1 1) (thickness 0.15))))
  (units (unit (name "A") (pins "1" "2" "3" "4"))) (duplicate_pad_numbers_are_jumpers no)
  (pad "1" thru_hole oval (at 0 0 90) (size 3 1.75) (drill 1) (layers "*.Cu" "*.Mask") (remove_unused_layers no) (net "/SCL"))
  (pad "2" thru_hole oval (at 0 2.54 90) (size 3 1.75) (drill 1) (layers "*.Cu" "*.Mask") (remove_unused_layers no) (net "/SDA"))
  (pad "3" thru_hole oval (at 0 5.08 90) (size 3 1.75) (drill 1) (layers "*.Cu" "*.Mask") (remove_unused_layers no) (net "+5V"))
  (pad "4" thru_hole oval (at 0 7.62 90) (size 3 1.75) (drill 1) (layers "*.Cu" "*.Mask") (remove_unused_layers no) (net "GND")))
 (gr_rect (start 146.25 66) (end 191.75 120) (stroke (width 0.05) (type solid)) (fill no) (layer "Edge.Cuts"))
 (segment (start 172.25 88.41) (end 172.25 98.25) (width 0.75) (layer "B.Cu") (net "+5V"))
 (segment (start 172.25 78.25) (end 172.25 86) (width 0.75) (layer "B.Cu") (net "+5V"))
 (segment (start 186.52 94.825) (end 186.52 90.25) (width 1) (layer "B.Cu") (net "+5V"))
 (segment (start 156.5 70.96) (end 161.44 70.96) (width 0.75) (layer "B.Cu") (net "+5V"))
 (segment (start 186.52 85.66) (end 186.52 90.25) (width 1) (layer "B.Cu") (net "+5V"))
 (segment (start 186.52 97.98) (end 186.52 94.825) (width 0.75) (layer "B.Cu") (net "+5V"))
 (segment (start 162.75 76.5) (end 170.5 76.5) (width 0.75) (layer "B.Cu") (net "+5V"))
 (segment (start 161.48 75.23) (end 162.75 76.5) (width 0.75) (layer "B.Cu") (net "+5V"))
 (segment (start 174 100) (end 184.5 100) (width 0.75) (layer "B.Cu") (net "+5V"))
 (segment (start 172.25 86) (end 173.455 87.205) (width 0.75) (layer "B.Cu") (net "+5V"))
 (segment (start 161.48 71) (end 167.225 71) (width 1) (layer "B.Cu") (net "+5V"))
 (segment (start 161.44 70.96) (end 161.48 71) (width 0.75) (layer "B.Cu") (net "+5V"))
 (segment (start 173.455 87.205) (end 172.25 88.41) (width 0.75) (layer "B.Cu") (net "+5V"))
 (segment (start 184.5 100) (end 186.52 97.98) (width 0.75) (layer "B.Cu") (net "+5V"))
 (segment (start 172.25 98.25) (end 174 100) (width 0.75) (layer "B.Cu") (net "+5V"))
 (segment (start 173.455 87.205) (end 176 87.205) (width 0.75) (layer "B.Cu") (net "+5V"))
 (segment (start 161.48 73.54) (end 161.48 75.23) (width 0.75) (layer "B.Cu") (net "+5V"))
 (segment (start 170.5 76.5) (end 172.25 78.25) (width 0.75) (layer "B.Cu") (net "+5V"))
 (segment (start 149.34 109.985) (end 149.42 110.065) (width 1) (layer "B.Cu") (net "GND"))
 (segment (start 149.42 105.08) (end 149.34 105) (width 1) (layer "B.Cu") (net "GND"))
 (segment (start 151.88 105) (end 151.88 109.985) (width 1) (layer "B.Cu") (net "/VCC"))
 (segment (start 151.875 75.375) (end 151.88 75.38) (width 0.75) (layer "B.Cu") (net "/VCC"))
 (segment (start 151.88 99.905) (end 151.88 94.865) (width 1) (layer "B.Cu") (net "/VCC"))
 (segment (start 151.88 105) (end 151.88 99.905) (width 1) (layer "B.Cu") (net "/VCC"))
 (segment (start 151.96 105.08) (end 151.88 105) (width 1) (layer "B.Cu") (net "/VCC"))
 (segment (start 151.88 109.985) (end 151.96 110.065) (width 1) (layer "B.Cu") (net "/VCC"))
 (segment (start 151.88 94.865) (end 151.88 90.25) (width 1) (layer "B.Cu") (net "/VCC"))
 (segment (start 156.5 73.5) (end 153.75 73.5) (width 0.75) (layer "B.Cu") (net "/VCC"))
 (segment (start 151.88 75.38) (end 151.88 90.25) (width 0.75) (layer "B.Cu") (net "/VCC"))
 (segment (start 153.75 73.5) (end 151.875 75.375) (width 0.75) (layer "B.Cu") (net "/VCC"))
 (segment (start 151.96 110.065) (end 151.96 115) (width 1) (layer "B.Cu") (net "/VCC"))
 (segment (start 158.785 92.285) (end 160.76 92.285) (width 1) (layer "B.Cu") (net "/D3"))
 (segment (start 156.75 90.25) (end 158.785 92.285) (width 1) (layer "B.Cu") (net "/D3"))
 (segment (start 154.42 90.25) (end 156.75 90.25) (width 1) (layer "B.Cu") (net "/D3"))
 (segment (start 158.895 112.605) (end 160.76 112.605) (width 1) (layer "B.Cu") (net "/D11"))
 (segment (start 154.5 115) (end 156.5 115) (width 1) (layer "B.Cu") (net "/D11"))
 (segment (start 156.5 115) (end 158.895 112.605) (width 1) (layer "B.Cu") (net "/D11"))
 (segment (start 154.42 105) (end 156 105) (width 1) (layer "B.Cu") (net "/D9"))
 (segment (start 158.525 107.525) (end 160.76 107.525) (width 1) (layer "B.Cu") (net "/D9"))
 (segment (start 156 105) (end 158.525 107.525) (width 1) (layer "B.Cu") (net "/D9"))
 (segment (start 176.07 112.43) (end 178.435 110.065) (width 1) (layer "B.Cu") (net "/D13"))
 (segment (start 178.435 110.065) (end 181.17 110.065) (width 1) (layer "B.Cu") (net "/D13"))
 (segment (start 176.07 115.075) (end 176.07 112.43) (width 1) (layer "B.Cu") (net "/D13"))
 (segment (start 176 115.145) (end 176.07 115.075) (width 1) (layer "B.Cu") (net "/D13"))
 (segment (start 160.76 115.145) (end 166.855 115.145) (width 0.75) (layer "B.Cu") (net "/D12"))
 (segment (start 166.855 115.145) (end 174.475 107.525) (width 0.75) (layer "B.Cu") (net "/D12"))
 (segment (start 174.475 107.525) (end 181.17 107.525) (width 0.75) (layer "B.Cu") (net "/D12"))
 (segment (start 160.76 104.985) (end 181.17 104.985) (width 0.75) (layer "B.Cu") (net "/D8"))
 (segment (start 158.995 89.745) (end 160.83 89.745) (width 1) (layer "B.Cu") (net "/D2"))
 (segment (start 158 88.75) (end 158.995 89.745) (width 1) (layer "B.Cu") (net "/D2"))
 (segment (start 154.67 85.58) (end 156.83 85.58) (width 1) (layer "B.Cu") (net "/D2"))
 (segment (start 156.83 85.58) (end 158 86.75) (width 1) (layer "B.Cu") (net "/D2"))
 (segment (start 158 86.75) (end 158 88.75) (width 1) (layer "B.Cu") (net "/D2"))
 (segment (start 164 85.25) (end 164 93.75) (width 0.75) (layer "B.Cu") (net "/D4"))
 (segment (start 154.67 83.04) (end 161.79 83.04) (width 0.75) (layer "B.Cu") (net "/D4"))
 (segment (start 161.79 83.04) (end 164 85.25) (width 0.75) (layer "B.Cu") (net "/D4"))
 (segment (start 164 93.75) (end 162.925 94.825) (width 0.75) (layer "B.Cu") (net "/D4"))
 (segment (start 162.925 94.825) (end 160.83 94.825) (width 0.75) (layer "B.Cu") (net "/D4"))
 (segment (start 154.42 94.865) (end 156.365 94.865) (width 1) (layer "B.Cu") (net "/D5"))
 (segment (start 158.865 97.365) (end 160.76 97.365) (width 1) (layer "B.Cu") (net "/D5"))
 (segment (start 156.365 94.865) (end 158.865 97.365) (width 1) (layer "B.Cu") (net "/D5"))
 (segment (start 154.42 99.905) (end 160.76 99.905) (width 1) (layer "B.Cu") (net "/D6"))
 (segment (start 166 83.5) (end 166 99.75) (width 0.75) (layer "B.Cu") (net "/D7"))
 (segment (start 163 80.5) (end 166 83.5) (width 0.75) (layer "B.Cu") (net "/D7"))
 (segment (start 166 99.75) (end 163.305 102.445) (width 0.75) (layer "B.Cu") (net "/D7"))
 (segment (start 154.67 80.5) (end 163 80.5) (width 0.75) (layer "B.Cu") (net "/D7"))
 (segment (start 163.305 102.445) (end 160.83 102.445) (width 0.75) (layer "B.Cu") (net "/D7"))
 (segment (start 154.5 110.065) (end 160.76 110.065) (width 1) (layer "B.Cu") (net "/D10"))
 (segment (start 176 97.365) (end 182.885 97.365) (width 0.75) (layer "B.Cu") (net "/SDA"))
 (segment (start 183.98 85.66) (end 183.98 90.25) (width 1) (layer "B.Cu") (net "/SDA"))
 (segment (start 182.885 97.365) (end 183.98 96.27) (width 0.75) (layer "B.Cu") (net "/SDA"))
 (segment (start 183.98 96.27) (end 183.98 94.825) (width 0.75) (layer "B.Cu") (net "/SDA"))
 (segment (start 183.98 90.25) (end 183.98 94.825) (width 1) (layer "B.Cu") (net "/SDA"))
 (segment (start 181.44 94.825) (end 181.44 90.25) (width 1) (layer "B.Cu") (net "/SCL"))
 (segment (start 181.44 85.66) (end 181.44 90.25) (width 1) (layer "B.Cu") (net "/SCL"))
 (segment (start 176 94.825) (end 181.44 94.825) (width 1) (layer "B.Cu") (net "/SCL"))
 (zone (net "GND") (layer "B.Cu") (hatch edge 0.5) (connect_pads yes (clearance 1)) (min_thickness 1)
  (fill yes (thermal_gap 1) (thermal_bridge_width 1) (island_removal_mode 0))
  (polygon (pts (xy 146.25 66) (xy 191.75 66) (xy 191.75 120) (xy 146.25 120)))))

